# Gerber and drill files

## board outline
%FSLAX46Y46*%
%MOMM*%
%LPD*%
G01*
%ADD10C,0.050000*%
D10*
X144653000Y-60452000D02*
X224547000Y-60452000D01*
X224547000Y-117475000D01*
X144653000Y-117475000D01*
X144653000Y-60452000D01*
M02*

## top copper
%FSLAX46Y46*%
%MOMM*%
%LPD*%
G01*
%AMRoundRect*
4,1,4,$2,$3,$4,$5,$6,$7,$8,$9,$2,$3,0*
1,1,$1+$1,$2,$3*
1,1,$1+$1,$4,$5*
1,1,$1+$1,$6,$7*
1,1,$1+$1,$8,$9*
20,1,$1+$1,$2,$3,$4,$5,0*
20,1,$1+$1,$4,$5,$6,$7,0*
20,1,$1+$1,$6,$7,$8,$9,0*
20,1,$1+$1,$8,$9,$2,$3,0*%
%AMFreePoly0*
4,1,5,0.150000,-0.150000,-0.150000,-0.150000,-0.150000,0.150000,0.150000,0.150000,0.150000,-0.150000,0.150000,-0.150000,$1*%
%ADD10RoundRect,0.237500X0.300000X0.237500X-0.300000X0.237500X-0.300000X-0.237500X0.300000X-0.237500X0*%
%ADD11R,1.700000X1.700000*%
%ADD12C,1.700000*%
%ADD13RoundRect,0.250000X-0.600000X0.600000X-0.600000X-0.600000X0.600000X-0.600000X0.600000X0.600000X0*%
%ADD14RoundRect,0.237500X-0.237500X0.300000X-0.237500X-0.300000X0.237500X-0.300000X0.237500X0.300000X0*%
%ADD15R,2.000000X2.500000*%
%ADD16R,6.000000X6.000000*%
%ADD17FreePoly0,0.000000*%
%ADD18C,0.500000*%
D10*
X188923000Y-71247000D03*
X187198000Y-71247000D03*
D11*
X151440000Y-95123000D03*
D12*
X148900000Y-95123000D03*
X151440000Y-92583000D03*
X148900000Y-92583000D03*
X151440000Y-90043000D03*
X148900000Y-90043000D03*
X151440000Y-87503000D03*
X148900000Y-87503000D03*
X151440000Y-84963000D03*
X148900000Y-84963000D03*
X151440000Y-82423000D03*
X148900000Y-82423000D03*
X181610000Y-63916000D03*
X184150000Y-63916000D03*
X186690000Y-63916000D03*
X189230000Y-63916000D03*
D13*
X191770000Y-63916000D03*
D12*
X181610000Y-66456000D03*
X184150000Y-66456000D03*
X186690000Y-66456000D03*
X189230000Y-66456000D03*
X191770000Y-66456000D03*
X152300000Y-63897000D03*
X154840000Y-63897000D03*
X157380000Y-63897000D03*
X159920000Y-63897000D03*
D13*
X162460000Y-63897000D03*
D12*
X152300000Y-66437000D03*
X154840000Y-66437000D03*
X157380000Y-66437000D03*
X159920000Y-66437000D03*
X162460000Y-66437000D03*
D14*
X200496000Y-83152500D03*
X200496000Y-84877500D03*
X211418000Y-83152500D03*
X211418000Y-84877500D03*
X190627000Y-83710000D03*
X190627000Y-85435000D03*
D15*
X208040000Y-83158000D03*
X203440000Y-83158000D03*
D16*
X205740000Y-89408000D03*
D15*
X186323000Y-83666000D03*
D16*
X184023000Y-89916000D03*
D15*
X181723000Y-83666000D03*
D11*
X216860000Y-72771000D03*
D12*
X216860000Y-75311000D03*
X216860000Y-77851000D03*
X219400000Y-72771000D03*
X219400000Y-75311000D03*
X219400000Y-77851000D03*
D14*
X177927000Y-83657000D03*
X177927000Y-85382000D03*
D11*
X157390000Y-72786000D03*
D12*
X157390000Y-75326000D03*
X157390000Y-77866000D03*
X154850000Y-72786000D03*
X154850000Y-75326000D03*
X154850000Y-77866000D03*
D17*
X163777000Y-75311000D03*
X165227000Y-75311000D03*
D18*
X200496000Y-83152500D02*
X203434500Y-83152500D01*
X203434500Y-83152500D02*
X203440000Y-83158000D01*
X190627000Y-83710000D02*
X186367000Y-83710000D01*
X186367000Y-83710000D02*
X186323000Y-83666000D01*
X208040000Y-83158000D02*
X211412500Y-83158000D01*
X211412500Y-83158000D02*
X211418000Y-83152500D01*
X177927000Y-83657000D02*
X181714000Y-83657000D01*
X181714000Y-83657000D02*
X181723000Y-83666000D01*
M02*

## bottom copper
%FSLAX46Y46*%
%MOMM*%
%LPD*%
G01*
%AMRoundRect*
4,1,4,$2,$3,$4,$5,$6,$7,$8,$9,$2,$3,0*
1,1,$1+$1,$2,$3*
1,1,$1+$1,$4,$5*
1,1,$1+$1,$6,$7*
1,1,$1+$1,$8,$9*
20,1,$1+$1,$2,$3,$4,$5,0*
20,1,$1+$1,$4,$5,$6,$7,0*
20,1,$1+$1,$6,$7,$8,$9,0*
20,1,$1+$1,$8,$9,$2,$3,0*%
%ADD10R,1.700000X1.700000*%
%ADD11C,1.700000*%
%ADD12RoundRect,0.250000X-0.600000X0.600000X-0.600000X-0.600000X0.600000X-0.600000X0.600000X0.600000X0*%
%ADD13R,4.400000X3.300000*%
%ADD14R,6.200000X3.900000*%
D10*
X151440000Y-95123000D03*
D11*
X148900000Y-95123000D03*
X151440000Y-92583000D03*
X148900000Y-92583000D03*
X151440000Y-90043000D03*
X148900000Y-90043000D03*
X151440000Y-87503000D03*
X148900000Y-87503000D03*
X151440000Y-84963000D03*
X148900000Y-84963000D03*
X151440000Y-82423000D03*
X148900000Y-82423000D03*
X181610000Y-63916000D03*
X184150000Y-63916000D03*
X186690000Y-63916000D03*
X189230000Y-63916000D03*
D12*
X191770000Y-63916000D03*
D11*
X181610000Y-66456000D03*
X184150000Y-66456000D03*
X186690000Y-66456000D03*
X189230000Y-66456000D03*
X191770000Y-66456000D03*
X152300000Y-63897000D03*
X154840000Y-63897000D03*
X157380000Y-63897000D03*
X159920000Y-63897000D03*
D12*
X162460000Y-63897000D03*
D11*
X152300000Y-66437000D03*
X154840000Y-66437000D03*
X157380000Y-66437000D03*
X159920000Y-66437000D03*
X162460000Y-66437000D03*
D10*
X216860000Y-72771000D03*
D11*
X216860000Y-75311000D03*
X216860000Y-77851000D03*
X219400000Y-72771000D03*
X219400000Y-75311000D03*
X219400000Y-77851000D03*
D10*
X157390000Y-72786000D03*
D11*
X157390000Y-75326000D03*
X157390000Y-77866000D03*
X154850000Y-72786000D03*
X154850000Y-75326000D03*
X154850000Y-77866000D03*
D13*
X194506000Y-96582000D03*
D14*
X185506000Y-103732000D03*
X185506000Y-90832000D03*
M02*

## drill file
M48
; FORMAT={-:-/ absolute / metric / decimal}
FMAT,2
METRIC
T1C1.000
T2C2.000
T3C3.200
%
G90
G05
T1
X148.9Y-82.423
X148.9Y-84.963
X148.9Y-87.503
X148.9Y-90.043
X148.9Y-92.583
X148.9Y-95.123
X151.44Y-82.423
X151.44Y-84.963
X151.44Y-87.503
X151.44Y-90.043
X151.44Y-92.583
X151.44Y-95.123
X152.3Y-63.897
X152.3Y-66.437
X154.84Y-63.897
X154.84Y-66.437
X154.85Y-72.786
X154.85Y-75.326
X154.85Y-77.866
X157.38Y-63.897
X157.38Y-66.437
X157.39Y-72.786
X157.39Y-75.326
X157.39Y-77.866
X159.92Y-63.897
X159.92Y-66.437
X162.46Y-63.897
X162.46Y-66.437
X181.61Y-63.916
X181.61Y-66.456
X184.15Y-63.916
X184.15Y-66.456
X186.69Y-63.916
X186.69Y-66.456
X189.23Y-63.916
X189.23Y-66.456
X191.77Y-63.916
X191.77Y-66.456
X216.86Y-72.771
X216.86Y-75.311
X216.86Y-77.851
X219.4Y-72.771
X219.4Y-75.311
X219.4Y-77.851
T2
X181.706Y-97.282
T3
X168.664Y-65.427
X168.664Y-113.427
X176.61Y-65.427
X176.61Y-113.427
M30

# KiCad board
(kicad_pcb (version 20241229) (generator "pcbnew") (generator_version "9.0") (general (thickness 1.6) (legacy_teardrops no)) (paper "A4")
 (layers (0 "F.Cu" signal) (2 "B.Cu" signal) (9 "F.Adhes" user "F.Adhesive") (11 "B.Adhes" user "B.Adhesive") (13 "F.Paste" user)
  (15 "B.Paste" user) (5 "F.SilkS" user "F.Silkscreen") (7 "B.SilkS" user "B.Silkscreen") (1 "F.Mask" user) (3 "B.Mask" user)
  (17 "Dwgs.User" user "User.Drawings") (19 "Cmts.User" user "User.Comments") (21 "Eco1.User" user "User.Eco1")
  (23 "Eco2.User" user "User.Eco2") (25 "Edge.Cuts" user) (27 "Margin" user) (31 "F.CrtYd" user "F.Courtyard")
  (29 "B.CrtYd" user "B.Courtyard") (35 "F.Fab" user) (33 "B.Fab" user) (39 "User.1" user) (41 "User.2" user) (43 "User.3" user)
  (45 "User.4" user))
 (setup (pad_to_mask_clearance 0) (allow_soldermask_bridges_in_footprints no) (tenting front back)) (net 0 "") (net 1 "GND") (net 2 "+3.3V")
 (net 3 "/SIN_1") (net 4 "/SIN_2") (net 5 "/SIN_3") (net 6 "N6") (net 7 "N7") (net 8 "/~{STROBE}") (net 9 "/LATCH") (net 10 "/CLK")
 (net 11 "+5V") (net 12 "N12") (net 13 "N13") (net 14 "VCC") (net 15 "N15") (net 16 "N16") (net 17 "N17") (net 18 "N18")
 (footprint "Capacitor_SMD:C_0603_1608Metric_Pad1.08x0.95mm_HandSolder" (layer "F.Cu") (at 188.0605 71.247 180)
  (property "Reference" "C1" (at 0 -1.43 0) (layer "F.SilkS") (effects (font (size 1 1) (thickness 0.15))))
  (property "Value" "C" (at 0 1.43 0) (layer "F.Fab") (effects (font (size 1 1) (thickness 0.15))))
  (pad "1" smd roundrect (at -0.8625 0 180) (size 1.075 0.95) (layers "F.Cu" "F.Mask" "F.Paste") (roundrect_rratio 0.25) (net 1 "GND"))
  (pad "2" smd roundrect (at 0.8625 0 180) (size 1.075 0.95) (layers "F.Cu" "F.Mask" "F.Paste") (roundrect_rratio 0.25) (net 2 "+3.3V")))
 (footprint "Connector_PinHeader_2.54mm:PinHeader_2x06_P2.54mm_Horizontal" (layer "F.Cu") (at 151.44 95.123 180)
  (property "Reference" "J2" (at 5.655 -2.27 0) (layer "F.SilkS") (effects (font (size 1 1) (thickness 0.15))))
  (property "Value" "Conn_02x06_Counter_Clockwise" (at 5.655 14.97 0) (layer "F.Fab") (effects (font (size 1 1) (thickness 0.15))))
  (pad "1" thru_hole rect (at 0 0 180) (size 1.7 1.7) (drill 1) (layers "*.Cu" "*.Mask") (remove_unused_layers no) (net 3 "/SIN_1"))
  (pad "2" thru_hole circle (at 2.54 0 180) (size 1.7 1.7) (drill 1) (layers "*.Cu" "*.Mask") (remove_unused_layers no) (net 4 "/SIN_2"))
  (pad "3" thru_hole circle (at 0 2.54 180) (size 1.7 1.7) (drill 1) (layers "*.Cu" "*.Mask") (remove_unused_layers no) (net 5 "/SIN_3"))
  (pad "4" thru_hole circle (at 2.54 2.54 180) (size 1.7 1.7) (drill 1) (layers "*.Cu" "*.Mask") (remove_unused_layers no) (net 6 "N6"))
  (pad "5" thru_hole circle (at 0 5.08 180) (size 1.7 1.7) (drill 1) (layers "*.Cu" "*.Mask") (remove_unused_layers no) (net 1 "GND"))
  (pad "6" thru_hole circle (at 2.54 5.08 180) (size 1.7 1.7) (drill 1) (layers "*.Cu" "*.Mask") (remove_unused_layers no) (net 2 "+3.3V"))
  (pad "7" thru_hole circle (at 0 7.62 180) (size 1.7 1.7) (drill 1) (layers "*.Cu" "*.Mask") (remove_unused_layers no) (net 2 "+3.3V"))
  (pad "8" thru_hole circle (at 2.54 7.62 180) (size 1.7 1.7) (drill 1) (layers "*.Cu" "*.Mask") (remove_unused_layers no) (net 1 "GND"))
  (pad "9" thru_hole circle (at 0 10.16 180) (size 1.7 1.7) (drill 1) (layers "*.Cu" "*.Mask") (remove_unused_layers no) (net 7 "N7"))
  (pad "10" thru_hole circle (at 2.54 10.16 180) (size 1.7 1.7) (drill 1) (layers "*.Cu" "*.Mask") (remove_unused_layers no)
   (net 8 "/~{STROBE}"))
  (pad "11" thru_hole circle (at 0 12.7 180) (size 1.7 1.7) (drill 1) (layers "*.Cu" "*.Mask") (remove_unused_layers no) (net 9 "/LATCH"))
  (pad "12" thru_hole circle (at 2.54 12.7 180) (size 1.7 1.7) (drill 1) (layers "*.Cu" "*.Mask") (remove_unused_layers no) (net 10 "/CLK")))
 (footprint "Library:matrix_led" (layer "F.Cu") (at 186.69 58.836)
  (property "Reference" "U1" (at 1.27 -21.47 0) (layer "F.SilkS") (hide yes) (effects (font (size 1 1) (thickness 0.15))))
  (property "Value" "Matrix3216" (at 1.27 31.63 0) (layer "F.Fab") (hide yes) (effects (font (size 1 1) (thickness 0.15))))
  (pad "1" thru_hole circle (at -5.08 5.08 270) (size 1.7 1.7) (drill 1) (layers "*.Cu" "*.Mask") (remove_unused_layers no) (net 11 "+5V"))
  (pad "2" thru_hole circle (at -2.54 5.08 270) (size 1.7 1.7) (drill 1) (layers "*.Cu" "*.Mask") (remove_unused_layers no) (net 3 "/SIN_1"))
  (pad "3" thru_hole circle (at 0 5.08 270) (size 1.7 1.7) (drill 1) (layers "*.Cu" "*.Mask") (remove_unused_layers no) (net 4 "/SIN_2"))
  (pad "4" thru_hole circle (at 2.54 5.08 270) (size 1.7 1.7) (drill 1) (layers "*.Cu" "*.Mask") (remove_unused_layers no) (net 5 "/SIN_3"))
  (pad "5" thru_hole roundrect (at 5.08 5.08 270) (size 1.7 1.7) (drill 1) (layers "*.Cu" "*.Mask") (remove_unused_layers no)
   (roundrect_rratio 0.147059) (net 10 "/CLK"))
  (pad "6" thru_hole circle (at -5.08 7.62 270) (size 1.7 1.7) (drill 1) (layers "*.Cu" "*.Mask") (remove_unused_layers no) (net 9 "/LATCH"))
  (pad "7" thru_hole circle (at -2.54 7.62 270) (size 1.7 1.7) (drill 1) (layers "*.Cu" "*.Mask") (remove_unused_layers no)
   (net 8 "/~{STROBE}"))
  (pad "8" thru_hole circle (at 0 7.62 270) (size 1.7 1.7) (drill 1) (layers "*.Cu" "*.Mask") (remove_unused_layers no) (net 2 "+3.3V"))
  (pad "9" thru_hole circle (at 2.54 7.62 270) (size 1.7 1.7) (drill 1) (layers "*.Cu" "*.Mask") (remove_unused_layers no) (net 1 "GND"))
  (pad "10" thru_hole circle (at 5.08 7.62 270) (size 1.7 1.7) (drill 1) (layers "*.Cu" "*.Mask") (remove_unused_layers no) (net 1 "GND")))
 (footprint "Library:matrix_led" (layer "F.Cu") (at 117.248 58.817)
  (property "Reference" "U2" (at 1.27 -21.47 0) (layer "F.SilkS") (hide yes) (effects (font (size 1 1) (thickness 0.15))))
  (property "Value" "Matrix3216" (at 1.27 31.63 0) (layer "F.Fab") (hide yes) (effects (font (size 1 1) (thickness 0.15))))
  (pad "31" thru_hole circle (at 35.052 5.08 270) (size 1.7 1.7) (drill 1) (layers "*.Cu" "*.Mask") (remove_unused_layers no) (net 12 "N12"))
  (pad "32" thru_hole circle (at 37.592 5.08 270) (size 1.7 1.7) (drill 1) (layers "*.Cu" "*.Mask") (remove_unused_layers no)
   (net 3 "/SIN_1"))
  (pad "33" thru_hole circle (at 40.132 5.08 270) (size 1.7 1.7) (drill 1) (layers "*.Cu" "*.Mask") (remove_unused_layers no)
   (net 4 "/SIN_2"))
  (pad "34" thru_hole circle (at 42.672 5.08 270) (size 1.7 1.7) (drill 1) (layers "*.Cu" "*.Mask") (remove_unused_layers no)
   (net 5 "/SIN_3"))
  (pad "35" thru_hole roundrect (at 45.212 5.08 270) (size 1.7 1.7) (drill 1) (layers "*.Cu" "*.Mask") (remove_unused_layers no)
   (roundrect_rratio 0.147059) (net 10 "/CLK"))
  (pad "36" thru_hole circle (at 35.052 7.62 270) (size 1.7 1.7) (drill 1) (layers "*.Cu" "*.Mask") (remove_unused_layers no)
   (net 9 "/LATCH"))
  (pad "37" thru_hole circle (at 37.592 7.62 270) (size 1.7 1.7) (drill 1) (layers "*.Cu" "*.Mask") (remove_unused_layers no)
   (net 8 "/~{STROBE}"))
  (pad "38" thru_hole circle (at 40.132 7.62 270) (size 1.7 1.7) (drill 1) (layers "*.Cu" "*.Mask") (remove_unused_layers no) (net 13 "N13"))
  (pad "39" thru_hole circle (at 42.672 7.62 270) (size 1.7 1.7) (drill 1) (layers "*.Cu" "*.Mask") (remove_unused_layers no) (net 1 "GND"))
  (pad "40" thru_hole circle (at 45.212 7.62 270) (size 1.7 1.7) (drill 1) (layers "*.Cu" "*.Mask") (remove_unused_layers no) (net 1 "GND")))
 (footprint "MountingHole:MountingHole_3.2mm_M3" (layer "F.Cu") (at 176.6098 65.4266)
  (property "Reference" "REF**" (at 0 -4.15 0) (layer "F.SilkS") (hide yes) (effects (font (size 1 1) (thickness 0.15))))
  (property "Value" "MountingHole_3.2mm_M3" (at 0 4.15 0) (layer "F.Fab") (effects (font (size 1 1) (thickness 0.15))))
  (pad "" np_thru_hole circle (at 0 0) (size 3.2 3.2) (drill 3.2) (layers "*.Cu" "*.Mask")))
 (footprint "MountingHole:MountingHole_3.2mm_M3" (layer "F.Cu") (at 168.664 65.4266)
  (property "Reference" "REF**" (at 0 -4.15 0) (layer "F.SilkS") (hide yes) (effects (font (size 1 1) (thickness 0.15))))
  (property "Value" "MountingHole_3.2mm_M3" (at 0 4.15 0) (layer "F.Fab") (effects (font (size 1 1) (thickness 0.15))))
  (pad "" np_thru_hole circle (at 0 0) (size 3.2 3.2) (drill 3.2) (layers "*.Cu" "*.Mask")))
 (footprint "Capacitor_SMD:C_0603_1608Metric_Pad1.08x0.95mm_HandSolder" (layer "F.Cu") (at 200.496 84.015 -90)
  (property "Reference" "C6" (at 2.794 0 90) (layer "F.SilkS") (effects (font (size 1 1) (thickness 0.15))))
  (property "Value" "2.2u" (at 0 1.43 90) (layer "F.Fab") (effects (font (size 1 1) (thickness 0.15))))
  (pad "1" smd roundrect (at -0.8625 0 270) (size 1.075 0.95) (layers "F.Cu" "F.Mask" "F.Paste") (roundrect_rratio 0.25) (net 2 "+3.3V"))
  (pad "2" smd roundrect (at 0.8625 0 270) (size 1.075 0.95) (layers "F.Cu" "F.Mask" "F.Paste") (roundrect_rratio 0.25) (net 1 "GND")))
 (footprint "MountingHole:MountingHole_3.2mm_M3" (layer "F.Cu") (at 176.6098 113.4266)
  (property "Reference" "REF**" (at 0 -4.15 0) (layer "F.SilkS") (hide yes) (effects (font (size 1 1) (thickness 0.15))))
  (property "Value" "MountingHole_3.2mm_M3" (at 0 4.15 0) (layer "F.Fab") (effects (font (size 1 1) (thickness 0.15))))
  (pad "" np_thru_hole circle (at 0 0) (size 3.2 3.2) (drill 3.2) (layers "*.Cu" "*.Mask")))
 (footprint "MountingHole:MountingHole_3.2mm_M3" (layer "F.Cu") (at 168.664 113.4266)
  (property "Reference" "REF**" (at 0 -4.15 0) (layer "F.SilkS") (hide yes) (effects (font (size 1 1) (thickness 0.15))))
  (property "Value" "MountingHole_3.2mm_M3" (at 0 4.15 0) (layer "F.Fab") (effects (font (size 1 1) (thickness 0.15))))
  (pad "" np_thru_hole circle (at 0 0) (size 3.2 3.2) (drill 3.2) (layers "*.Cu" "*.Mask")))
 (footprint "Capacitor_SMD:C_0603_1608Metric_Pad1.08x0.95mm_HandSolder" (layer "F.Cu") (at 211.418 84.015 -90)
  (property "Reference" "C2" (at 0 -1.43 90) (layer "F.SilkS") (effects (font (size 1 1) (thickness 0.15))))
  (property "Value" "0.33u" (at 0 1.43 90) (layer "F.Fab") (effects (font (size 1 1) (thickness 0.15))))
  (pad "1" smd roundrect (at -0.8625 0 270) (size 1.075 0.95) (layers "F.Cu" "F.Mask" "F.Paste") (roundrect_rratio 0.25) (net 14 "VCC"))
  (pad "2" smd roundrect (at 0.8625 0 270) (size 1.075 0.95) (layers "F.Cu" "F.Mask" "F.Paste") (roundrect_rratio 0.25) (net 1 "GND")))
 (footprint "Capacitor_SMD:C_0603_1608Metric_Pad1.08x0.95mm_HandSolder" (layer "F.Cu") (at 190.627 84.5725 -90)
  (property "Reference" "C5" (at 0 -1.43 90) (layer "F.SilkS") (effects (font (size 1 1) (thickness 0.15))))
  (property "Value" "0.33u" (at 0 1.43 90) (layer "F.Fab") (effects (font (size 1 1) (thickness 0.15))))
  (pad "1" smd roundrect (at -0.8625 0 270) (size 1.075 0.95) (layers "F.Cu" "F.Mask" "F.Paste") (roundrect_rratio 0.25) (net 14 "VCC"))
  (pad "2" smd roundrect (at 0.8625 0 270) (size 1.075 0.95) (layers "F.Cu" "F.Mask" "F.Paste") (roundrect_rratio 0.25) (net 1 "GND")))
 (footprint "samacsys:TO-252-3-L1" (layer "F.Cu") (at 205.74 91.208 180)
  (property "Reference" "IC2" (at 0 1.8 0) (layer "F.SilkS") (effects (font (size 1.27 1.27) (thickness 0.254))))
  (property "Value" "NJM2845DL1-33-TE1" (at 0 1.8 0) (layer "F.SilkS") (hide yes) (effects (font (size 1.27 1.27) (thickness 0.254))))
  (pad "1" smd rect (at -2.3 8.05 180) (size 2 2.5) (layers "F.Cu" "F.Mask" "F.Paste") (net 14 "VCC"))
  (pad "2" smd rect (at 2.3 8.05 180) (size 2 2.5) (layers "F.Cu" "F.Mask" "F.Paste") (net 2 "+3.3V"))
  (pad "3" smd rect (at 0 1.8 270) (size 6 6) (layers "F.Cu" "F.Mask" "F.Paste") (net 1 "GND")))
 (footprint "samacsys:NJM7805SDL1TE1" (layer "F.Cu") (at 184.023 87.721 180)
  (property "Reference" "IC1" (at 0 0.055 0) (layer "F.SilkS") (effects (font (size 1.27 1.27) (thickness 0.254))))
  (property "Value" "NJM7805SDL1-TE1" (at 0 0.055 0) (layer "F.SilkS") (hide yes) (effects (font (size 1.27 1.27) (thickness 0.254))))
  (pad "1" smd rect (at -2.3 4.055 180) (size 2 2.5) (layers "F.Cu" "F.Mask" "F.Paste") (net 14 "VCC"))
  (pad "2" smd rect (at 0 -2.195 270) (size 6 6) (layers "F.Cu" "F.Mask" "F.Paste") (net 1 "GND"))
  (pad "3" smd rect (at 2.3 4.055 180) (size 2 2.5) (layers "F.Cu" "F.Mask" "F.Paste") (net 11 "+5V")))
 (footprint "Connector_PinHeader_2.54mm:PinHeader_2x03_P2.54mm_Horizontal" (layer "F.Cu") (at 216.86 72.771)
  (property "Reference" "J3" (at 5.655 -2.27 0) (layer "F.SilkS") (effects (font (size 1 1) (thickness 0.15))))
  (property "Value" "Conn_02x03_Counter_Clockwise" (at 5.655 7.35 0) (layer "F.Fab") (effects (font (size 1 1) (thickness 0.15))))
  (pad "1" thru_hole rect (at 0 0) (size 1.7 1.7) (drill 1) (layers "*.Cu" "*.Mask") (remove_unused_layers no) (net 1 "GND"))
  (pad "2" thru_hole circle (at 0 2.54) (size 1.7 1.7) (drill 1) (layers "*.Cu" "*.Mask") (remove_unused_layers no) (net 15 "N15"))
  (pad "3" thru_hole circle (at 0 5.08) (size 1.7 1.7) (drill 1) (layers "*.Cu" "*.Mask") (remove_unused_layers no) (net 14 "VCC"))
  (pad "4" thru_hole circle (at 2.54 0) (size 1.7 1.7) (drill 1) (layers "*.Cu" "*.Mask") (remove_unused_layers no) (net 14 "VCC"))
  (pad "5" thru_hole circle (at 2.54 2.54) (size 1.7 1.7) (drill 1) (layers "*.Cu" "*.Mask") (remove_unused_layers no) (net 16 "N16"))
  (pad "6" thru_hole circle (at 2.54 5.08) (size 1.7 1.7) (drill 1) (layers "*.Cu" "*.Mask") (remove_unused_layers no) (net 1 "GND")))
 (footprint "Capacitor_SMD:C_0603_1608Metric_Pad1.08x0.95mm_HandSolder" (layer "F.Cu") (at 177.927 84.5195 -90)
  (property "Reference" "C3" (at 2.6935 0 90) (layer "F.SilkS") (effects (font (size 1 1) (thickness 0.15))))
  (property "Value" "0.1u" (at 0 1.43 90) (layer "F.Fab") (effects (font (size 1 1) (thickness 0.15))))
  (pad "1" smd roundrect (at -0.8625 0 270) (size 1.075 0.95) (layers "F.Cu" "F.Mask" "F.Paste") (roundrect_rratio 0.25) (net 11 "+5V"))
  (pad "2" smd roundrect (at 0.8625 0 270) (size 1.075 0.95) (layers "F.Cu" "F.Mask" "F.Paste") (roundrect_rratio 0.25) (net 1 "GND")))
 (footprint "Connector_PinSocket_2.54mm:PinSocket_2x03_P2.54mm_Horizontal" (layer "F.Cu") (at 157.39 72.786)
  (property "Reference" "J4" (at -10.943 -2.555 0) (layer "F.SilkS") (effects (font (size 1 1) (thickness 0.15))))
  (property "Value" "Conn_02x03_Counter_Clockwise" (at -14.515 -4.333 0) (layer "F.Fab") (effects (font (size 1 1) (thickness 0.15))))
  (pad "1" thru_hole rect (at 0 0) (size 1.7 1.7) (drill 1) (layers "*.Cu" "*.Mask") (remove_unused_layers no) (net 1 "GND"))
  (pad "2" thru_hole circle (at 0 2.54) (size 1.7 1.7) (drill 1) (layers "*.Cu" "*.Mask") (remove_unused_layers no) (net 2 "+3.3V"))
  (pad "3" thru_hole circle (at 0 5.08) (size 1.7 1.7) (drill 1) (layers "*.Cu" "*.Mask") (remove_unused_layers no) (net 14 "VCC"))
  (pad "4" thru_hole circle (at -2.54 0) (size 1.7 1.7) (drill 1) (layers "*.Cu" "*.Mask") (remove_unused_layers no) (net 14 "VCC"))
  (pad "5" thru_hole circle (at -2.54 2.54) (size 1.7 1.7) (drill 1) (layers "*.Cu" "*.Mask") (remove_unused_layers no) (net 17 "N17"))
  (pad "6" thru_hole circle (at -2.54 5.08) (size 1.7 1.7) (drill 1) (layers "*.Cu" "*.Mask") (remove_unused_layers no) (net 1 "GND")))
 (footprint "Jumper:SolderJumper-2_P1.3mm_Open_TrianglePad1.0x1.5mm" (layer "F.Cu") (at 164.502 75.311)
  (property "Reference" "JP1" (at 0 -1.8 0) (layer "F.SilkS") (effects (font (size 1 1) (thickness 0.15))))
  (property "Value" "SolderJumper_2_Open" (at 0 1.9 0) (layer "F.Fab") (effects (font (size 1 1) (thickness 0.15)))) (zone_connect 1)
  (pad "1" smd custom (at -0.725 0) (size 0.3 0.3) (layers "F.Cu" "F.Mask") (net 2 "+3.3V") (zone_connect 2) (thermal_bridge_angle 45)
   (options (clearance outline) (anchor rect)) (primitives))
  (pad "2" smd custom (at 0.725 0) (size 0.3 0.3) (layers "F.Cu" "F.Mask") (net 15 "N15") (zone_connect 2) (thermal_bridge_angle 45)
   (options (clearance outline) (anchor rect)) (primitives)))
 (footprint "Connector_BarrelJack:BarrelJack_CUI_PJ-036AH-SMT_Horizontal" (layer "B.Cu") (at 188.706 97.282 90)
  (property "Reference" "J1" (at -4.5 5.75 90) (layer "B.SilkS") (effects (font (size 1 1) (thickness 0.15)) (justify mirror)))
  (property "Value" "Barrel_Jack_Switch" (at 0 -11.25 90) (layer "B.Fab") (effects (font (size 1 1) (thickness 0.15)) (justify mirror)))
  (pad "" np_thru_hole circle (at 0 -7 90) (size 2 2) (drill 2) (layers "*.Cu" "*.Mask"))
  (pad "1" smd rect (at 0.7 5.8 90) (size 3.3 4.4) (layers "B.Cu" "B.Mask" "B.Paste") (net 14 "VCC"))
  (pad "2" smd rect (at -6.45 -3.2 90) (size 3.9 6.2) (layers "B.Cu" "B.Mask" "B.Paste") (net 1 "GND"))
  (pad "3" smd rect (at 6.45 -3.2 90) (size 3.9 6.2) (layers "B.Cu" "B.Mask" "B.Paste") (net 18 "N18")))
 (gr_rect (start 144.653 60.452) (end 224.547 117.475) (stroke (width 0.05) (type solid)) (fill no) (layer "Edge.Cuts"))
 (segment (start 200.496 83.1525) (end 203.4345 83.1525) (width 0.5) (layer "F.Cu") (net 2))
 (segment (start 203.4345 83.1525) (end 203.44 83.158) (width 0.5) (layer "F.Cu") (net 2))
 (segment (start 190.627 83.71) (end 186.367 83.71) (width 0.5) (layer "F.Cu") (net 14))
 (segment (start 186.367 83.71) (end 186.323 83.666) (width 0.5) (layer "F.Cu") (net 14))
 (segment (start 208.04 83.158) (end 211.4125 83.158) (width 0.5) (layer "F.Cu") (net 14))
 (segment (start 211.4125 83.158) (end 211.418 83.1525) (width 0.5) (layer "F.Cu") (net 14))
 (segment (start 177.927 83.657) (end 181.714 83.657) (width 0.5) (layer "F.Cu") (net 11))
 (segment (start 181.714 83.657) (end 181.723 83.666) (width 0.5) (layer "F.Cu") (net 11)))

